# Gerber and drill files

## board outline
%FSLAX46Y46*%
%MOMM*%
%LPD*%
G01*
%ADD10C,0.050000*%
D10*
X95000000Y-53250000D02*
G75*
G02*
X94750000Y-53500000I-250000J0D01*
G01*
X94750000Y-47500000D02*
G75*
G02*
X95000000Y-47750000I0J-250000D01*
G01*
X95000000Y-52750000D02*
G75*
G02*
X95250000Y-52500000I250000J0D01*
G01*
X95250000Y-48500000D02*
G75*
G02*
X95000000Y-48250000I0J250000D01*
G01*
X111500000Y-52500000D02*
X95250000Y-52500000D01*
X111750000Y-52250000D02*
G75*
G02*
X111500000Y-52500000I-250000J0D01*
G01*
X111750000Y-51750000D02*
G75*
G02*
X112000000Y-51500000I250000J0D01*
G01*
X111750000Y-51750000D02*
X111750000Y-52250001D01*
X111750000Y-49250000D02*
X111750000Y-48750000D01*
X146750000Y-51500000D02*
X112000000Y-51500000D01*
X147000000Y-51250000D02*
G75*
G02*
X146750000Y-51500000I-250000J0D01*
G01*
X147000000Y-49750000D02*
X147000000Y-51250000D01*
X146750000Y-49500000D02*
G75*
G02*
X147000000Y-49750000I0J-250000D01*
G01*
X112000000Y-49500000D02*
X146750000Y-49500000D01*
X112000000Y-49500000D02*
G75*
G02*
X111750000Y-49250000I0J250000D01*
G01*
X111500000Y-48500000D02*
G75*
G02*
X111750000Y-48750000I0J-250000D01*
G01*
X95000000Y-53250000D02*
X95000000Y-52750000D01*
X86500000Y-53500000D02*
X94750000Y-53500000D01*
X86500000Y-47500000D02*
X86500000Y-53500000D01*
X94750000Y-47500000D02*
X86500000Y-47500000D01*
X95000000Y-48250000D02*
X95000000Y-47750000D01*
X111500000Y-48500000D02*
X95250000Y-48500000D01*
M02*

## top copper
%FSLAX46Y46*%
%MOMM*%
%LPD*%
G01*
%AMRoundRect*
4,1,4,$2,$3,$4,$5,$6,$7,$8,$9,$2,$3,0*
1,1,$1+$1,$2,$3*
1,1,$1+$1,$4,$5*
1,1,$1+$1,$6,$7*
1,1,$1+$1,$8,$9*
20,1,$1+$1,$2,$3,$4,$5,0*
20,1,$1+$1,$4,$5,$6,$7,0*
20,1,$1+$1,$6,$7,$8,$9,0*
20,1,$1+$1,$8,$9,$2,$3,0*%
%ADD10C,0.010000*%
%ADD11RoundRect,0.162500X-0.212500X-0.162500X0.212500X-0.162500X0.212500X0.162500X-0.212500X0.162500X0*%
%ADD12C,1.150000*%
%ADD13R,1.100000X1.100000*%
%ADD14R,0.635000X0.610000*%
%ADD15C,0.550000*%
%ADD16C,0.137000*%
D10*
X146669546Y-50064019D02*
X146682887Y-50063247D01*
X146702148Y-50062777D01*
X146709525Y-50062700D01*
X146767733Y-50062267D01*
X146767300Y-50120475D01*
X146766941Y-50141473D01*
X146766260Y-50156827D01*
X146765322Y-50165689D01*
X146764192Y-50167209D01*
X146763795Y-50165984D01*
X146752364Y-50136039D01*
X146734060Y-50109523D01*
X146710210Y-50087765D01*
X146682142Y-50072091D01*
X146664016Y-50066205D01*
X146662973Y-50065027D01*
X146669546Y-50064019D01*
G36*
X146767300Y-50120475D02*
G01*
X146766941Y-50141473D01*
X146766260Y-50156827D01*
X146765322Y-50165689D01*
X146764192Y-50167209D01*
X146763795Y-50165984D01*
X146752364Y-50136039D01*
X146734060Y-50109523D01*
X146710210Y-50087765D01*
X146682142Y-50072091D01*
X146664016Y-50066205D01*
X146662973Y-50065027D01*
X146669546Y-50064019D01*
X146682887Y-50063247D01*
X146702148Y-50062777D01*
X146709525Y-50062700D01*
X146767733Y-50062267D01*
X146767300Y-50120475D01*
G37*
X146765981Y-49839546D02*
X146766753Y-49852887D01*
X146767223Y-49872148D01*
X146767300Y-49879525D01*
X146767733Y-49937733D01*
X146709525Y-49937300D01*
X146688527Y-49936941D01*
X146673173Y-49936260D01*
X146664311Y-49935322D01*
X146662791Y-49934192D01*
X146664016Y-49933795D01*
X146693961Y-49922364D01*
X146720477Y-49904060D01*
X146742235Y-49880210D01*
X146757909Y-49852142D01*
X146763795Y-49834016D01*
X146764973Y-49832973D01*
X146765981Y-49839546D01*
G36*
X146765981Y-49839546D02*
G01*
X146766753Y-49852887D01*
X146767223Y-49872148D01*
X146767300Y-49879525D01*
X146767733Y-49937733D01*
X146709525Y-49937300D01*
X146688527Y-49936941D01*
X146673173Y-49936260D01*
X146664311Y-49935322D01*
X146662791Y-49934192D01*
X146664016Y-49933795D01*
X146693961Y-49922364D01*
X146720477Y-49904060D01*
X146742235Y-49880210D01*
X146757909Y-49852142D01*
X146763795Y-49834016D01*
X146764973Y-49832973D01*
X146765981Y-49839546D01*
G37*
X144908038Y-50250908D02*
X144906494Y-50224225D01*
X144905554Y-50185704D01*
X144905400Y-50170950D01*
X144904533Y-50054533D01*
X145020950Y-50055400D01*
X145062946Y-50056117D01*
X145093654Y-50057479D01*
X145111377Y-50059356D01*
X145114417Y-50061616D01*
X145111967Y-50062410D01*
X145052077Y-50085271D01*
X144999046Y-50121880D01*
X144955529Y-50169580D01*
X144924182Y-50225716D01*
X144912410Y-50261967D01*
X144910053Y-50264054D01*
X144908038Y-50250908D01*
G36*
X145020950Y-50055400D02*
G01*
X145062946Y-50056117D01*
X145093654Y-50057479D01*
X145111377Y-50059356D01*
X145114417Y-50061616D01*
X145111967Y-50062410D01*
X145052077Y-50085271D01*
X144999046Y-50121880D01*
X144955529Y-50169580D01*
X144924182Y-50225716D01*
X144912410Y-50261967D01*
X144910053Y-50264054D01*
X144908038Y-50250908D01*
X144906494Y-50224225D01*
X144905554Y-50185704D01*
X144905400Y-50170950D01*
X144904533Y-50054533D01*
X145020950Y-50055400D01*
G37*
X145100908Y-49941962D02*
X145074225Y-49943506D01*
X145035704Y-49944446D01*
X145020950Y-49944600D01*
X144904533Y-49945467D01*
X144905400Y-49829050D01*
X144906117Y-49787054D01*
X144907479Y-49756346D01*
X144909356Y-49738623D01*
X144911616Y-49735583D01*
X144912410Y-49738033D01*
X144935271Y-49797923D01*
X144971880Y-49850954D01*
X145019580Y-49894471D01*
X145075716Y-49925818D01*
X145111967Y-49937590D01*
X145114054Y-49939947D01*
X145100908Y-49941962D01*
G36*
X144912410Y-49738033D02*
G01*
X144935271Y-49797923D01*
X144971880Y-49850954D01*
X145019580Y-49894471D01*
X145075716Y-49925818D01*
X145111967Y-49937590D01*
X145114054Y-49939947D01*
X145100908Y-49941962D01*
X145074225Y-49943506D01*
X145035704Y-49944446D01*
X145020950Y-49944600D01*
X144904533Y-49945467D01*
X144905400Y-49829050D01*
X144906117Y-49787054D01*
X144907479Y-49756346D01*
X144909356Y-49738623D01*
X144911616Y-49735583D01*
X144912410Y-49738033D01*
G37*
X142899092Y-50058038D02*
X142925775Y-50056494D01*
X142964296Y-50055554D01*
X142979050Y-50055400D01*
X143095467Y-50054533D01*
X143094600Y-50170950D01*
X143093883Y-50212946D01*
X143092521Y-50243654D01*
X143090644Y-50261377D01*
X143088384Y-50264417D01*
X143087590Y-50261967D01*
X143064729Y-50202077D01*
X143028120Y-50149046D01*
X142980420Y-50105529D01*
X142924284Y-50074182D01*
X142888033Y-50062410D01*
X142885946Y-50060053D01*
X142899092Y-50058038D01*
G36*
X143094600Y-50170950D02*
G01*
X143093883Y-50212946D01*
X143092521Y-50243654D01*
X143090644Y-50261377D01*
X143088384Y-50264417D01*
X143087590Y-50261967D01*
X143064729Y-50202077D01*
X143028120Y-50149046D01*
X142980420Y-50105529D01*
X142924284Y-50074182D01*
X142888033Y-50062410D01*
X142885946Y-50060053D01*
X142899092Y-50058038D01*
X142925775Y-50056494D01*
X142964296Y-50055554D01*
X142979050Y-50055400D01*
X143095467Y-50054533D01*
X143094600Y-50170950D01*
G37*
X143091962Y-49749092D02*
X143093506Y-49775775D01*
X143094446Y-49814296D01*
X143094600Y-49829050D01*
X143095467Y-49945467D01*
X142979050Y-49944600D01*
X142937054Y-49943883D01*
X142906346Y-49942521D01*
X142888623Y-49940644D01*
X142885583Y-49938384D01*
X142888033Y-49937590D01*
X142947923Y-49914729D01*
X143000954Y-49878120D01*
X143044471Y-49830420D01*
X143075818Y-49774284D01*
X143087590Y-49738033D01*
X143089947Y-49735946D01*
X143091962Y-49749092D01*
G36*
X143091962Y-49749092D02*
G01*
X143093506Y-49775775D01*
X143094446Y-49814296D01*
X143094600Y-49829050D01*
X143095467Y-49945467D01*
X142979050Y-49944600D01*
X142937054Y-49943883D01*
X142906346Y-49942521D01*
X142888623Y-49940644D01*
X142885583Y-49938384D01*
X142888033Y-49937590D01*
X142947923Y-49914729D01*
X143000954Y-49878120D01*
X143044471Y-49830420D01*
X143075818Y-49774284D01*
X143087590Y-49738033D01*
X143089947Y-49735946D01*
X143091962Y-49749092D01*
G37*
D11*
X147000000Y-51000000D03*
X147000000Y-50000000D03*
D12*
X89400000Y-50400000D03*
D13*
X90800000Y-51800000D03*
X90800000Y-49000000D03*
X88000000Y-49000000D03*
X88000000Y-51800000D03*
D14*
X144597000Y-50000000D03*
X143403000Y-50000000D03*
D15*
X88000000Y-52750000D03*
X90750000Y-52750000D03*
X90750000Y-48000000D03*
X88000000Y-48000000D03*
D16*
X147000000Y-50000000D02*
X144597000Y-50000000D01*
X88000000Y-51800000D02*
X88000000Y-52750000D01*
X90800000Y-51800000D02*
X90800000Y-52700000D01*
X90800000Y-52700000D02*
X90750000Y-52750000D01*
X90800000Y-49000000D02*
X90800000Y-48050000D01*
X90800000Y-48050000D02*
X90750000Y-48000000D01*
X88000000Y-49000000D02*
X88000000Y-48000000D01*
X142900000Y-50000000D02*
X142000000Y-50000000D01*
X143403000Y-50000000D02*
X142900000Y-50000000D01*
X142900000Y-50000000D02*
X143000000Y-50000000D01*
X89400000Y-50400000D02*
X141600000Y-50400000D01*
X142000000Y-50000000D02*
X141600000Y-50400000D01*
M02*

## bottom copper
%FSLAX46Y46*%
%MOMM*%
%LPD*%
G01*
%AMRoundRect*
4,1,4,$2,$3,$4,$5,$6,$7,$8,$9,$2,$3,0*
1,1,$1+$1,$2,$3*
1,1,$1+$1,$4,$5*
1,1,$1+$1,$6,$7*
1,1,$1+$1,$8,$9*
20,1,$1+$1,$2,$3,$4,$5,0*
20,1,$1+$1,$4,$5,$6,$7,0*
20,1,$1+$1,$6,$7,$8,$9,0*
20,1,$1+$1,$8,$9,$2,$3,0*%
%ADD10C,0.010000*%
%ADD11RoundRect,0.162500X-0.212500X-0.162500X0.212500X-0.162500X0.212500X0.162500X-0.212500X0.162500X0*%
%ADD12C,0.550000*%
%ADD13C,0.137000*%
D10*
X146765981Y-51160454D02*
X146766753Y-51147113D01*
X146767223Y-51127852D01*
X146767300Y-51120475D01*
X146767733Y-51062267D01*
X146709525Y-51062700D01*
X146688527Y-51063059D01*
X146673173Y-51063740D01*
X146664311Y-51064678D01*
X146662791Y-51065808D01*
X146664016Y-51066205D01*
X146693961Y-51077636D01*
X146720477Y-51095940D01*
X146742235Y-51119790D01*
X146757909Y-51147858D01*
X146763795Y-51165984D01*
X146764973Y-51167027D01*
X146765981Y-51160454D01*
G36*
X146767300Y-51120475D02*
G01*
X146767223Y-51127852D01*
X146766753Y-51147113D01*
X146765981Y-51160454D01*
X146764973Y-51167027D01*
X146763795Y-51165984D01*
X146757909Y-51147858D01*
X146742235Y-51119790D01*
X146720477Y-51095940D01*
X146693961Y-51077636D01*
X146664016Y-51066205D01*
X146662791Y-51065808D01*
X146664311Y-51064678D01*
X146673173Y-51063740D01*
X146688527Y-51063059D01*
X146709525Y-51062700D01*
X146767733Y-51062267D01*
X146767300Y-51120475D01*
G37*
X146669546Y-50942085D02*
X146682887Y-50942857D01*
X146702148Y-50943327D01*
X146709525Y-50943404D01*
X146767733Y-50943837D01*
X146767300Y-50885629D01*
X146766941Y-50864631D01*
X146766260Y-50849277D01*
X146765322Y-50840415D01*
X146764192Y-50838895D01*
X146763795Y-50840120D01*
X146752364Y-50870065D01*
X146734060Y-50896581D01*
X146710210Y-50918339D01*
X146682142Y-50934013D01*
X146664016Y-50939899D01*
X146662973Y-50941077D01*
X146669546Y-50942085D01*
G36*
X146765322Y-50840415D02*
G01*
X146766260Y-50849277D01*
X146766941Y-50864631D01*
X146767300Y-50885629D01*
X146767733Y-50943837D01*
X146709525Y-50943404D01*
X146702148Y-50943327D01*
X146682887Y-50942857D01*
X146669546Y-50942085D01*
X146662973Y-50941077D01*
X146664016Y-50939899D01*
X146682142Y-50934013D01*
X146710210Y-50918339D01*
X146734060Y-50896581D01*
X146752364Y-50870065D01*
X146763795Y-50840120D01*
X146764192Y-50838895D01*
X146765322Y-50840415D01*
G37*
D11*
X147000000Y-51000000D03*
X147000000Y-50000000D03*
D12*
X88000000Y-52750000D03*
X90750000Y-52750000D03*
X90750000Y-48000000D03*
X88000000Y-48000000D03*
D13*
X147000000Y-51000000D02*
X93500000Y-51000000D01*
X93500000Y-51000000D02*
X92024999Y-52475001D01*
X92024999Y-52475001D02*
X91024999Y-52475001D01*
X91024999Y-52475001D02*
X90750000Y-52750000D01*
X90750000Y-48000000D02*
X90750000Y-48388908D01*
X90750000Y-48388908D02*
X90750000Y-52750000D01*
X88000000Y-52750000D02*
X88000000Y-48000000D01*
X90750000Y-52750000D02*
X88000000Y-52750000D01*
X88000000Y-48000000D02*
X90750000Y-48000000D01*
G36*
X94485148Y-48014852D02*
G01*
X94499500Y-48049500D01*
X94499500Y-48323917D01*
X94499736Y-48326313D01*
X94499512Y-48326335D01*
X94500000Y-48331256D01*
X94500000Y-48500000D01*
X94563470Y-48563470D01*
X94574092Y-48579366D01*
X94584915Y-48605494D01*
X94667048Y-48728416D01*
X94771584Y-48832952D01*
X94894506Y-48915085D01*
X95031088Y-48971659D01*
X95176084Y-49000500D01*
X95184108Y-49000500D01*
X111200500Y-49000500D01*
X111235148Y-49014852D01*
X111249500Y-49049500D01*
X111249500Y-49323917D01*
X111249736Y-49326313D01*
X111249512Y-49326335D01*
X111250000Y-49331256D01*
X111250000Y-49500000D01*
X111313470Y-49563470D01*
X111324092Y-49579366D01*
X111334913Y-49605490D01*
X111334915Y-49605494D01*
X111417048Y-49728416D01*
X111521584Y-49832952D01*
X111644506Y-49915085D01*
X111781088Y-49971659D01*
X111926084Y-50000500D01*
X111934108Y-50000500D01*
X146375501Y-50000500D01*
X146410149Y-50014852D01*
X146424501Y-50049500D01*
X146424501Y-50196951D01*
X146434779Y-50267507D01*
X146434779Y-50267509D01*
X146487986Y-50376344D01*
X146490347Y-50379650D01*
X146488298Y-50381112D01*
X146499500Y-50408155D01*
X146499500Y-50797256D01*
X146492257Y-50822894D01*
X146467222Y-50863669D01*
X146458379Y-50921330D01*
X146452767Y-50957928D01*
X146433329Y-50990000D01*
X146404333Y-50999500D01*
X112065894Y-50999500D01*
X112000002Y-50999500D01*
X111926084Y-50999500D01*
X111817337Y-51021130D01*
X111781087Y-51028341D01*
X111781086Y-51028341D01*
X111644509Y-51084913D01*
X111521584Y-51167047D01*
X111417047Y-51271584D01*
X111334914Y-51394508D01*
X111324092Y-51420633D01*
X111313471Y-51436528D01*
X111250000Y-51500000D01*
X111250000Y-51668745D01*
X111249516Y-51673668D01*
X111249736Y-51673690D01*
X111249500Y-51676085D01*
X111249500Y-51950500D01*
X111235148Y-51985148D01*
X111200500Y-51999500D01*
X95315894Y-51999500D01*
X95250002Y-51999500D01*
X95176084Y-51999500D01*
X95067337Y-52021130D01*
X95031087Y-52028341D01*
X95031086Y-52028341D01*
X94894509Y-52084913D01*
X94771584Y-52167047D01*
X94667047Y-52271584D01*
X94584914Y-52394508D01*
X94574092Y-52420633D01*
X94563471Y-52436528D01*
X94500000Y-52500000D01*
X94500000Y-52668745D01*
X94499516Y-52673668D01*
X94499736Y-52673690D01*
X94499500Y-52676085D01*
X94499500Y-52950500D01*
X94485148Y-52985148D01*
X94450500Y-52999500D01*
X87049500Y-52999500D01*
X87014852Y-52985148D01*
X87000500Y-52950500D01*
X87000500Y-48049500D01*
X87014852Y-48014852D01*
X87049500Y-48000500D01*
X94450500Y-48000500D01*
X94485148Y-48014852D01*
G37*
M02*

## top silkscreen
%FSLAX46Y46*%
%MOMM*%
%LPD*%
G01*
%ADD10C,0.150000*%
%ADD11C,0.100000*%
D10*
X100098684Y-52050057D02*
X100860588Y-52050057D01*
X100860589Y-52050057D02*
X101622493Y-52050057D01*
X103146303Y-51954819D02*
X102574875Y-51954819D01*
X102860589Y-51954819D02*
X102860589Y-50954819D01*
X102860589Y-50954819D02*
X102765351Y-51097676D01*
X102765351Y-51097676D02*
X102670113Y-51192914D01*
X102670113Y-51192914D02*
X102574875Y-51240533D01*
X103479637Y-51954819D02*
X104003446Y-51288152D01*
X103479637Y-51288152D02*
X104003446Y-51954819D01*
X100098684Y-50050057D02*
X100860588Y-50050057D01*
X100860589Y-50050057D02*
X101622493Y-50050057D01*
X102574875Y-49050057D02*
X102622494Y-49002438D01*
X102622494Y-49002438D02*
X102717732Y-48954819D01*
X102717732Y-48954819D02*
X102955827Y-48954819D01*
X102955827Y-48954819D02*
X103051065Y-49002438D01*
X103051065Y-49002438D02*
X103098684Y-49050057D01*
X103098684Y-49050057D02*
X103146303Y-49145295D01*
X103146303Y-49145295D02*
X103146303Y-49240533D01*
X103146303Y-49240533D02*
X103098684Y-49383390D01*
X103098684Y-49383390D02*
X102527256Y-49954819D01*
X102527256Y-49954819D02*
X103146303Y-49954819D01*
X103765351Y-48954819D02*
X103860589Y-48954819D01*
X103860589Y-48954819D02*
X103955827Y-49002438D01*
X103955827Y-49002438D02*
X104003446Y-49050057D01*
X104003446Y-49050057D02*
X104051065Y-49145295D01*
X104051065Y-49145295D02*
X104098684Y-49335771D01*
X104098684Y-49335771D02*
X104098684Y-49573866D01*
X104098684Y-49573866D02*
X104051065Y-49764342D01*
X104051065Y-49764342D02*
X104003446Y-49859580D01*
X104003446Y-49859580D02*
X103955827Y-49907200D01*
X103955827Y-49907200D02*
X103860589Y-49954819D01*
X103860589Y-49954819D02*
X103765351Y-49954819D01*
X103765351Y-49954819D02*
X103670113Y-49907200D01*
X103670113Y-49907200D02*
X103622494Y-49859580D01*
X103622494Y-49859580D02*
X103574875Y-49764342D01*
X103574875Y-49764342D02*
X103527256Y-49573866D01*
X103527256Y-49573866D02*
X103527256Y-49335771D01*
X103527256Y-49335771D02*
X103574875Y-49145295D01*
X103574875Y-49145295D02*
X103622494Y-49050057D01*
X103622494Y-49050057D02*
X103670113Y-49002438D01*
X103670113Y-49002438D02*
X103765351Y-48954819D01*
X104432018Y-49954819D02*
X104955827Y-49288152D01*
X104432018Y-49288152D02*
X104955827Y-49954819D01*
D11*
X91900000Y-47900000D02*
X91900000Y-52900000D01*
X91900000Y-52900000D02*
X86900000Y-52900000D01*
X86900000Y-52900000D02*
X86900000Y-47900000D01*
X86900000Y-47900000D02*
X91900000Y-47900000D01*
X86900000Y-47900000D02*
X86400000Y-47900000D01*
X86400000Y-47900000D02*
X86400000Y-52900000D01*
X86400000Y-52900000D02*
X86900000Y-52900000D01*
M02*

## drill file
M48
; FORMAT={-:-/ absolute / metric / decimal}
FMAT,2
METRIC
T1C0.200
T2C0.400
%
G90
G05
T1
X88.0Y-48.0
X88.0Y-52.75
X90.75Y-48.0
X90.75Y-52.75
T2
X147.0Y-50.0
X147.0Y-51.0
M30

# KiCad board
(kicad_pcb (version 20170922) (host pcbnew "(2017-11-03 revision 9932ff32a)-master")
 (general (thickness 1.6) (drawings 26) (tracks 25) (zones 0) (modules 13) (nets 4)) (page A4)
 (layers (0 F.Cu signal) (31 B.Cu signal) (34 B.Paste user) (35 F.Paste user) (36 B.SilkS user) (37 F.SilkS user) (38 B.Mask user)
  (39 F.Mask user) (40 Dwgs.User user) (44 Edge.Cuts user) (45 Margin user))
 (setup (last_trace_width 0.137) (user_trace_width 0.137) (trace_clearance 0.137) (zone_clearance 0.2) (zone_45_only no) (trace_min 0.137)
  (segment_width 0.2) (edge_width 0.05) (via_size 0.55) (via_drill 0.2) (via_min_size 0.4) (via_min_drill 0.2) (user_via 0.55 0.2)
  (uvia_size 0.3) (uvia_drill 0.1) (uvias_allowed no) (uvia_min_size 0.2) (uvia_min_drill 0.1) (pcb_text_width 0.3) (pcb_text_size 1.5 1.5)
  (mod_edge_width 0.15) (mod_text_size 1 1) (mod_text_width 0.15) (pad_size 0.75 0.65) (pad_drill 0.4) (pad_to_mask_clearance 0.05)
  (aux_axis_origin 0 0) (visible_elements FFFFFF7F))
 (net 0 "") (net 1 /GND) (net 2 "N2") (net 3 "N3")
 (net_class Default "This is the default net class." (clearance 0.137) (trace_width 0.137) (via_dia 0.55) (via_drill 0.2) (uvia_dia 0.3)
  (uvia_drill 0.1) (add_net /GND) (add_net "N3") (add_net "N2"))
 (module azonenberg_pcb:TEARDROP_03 (layer B.Cu) (at 146.7 51.13)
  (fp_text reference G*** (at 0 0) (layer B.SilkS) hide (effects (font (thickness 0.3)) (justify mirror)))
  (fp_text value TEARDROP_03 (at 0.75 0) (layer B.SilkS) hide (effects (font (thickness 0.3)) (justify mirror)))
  (fp_poly
   (pts (xy 0.065981 0.030454) (xy 0.066753 0.017113) (xy 0.067223 -0.002148) (xy 0.0673 -0.009525) (xy 0.067733 -0.067733)
    (xy 0.009525 -0.0673) (xy -0.011473 -0.066941) (xy -0.026827 -0.06626) (xy -0.035689 -0.065322) (xy -0.037209 -0.064192)
    (xy -0.035984 -0.063795) (xy -0.006039 -0.052364) (xy 0.020477 -0.03406) (xy 0.042235 -0.01021) (xy 0.057909 0.017858)
    (xy 0.063795 0.035984) (xy 0.064973 0.037027) (xy 0.065981 0.030454))
   (layer B.Cu) (width 0.01)))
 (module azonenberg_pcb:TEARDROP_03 (layer B.Cu) (at 146.7 50.876104 270)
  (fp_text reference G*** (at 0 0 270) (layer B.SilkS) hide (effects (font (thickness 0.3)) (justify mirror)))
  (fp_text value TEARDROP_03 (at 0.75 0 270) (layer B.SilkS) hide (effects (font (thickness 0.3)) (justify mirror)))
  (fp_poly
   (pts (xy 0.065981 0.030454) (xy 0.066753 0.017113) (xy 0.067223 -0.002148) (xy 0.0673 -0.009525) (xy 0.067733 -0.067733)
    (xy 0.009525 -0.0673) (xy -0.011473 -0.066941) (xy -0.026827 -0.06626) (xy -0.035689 -0.065322) (xy -0.037209 -0.064192)
    (xy -0.035984 -0.063795) (xy -0.006039 -0.052364) (xy 0.020477 -0.03406) (xy 0.042235 -0.01021) (xy 0.057909 0.017858)
    (xy 0.063795 0.035984) (xy 0.064973 0.037027) (xy 0.065981 0.030454))
   (layer B.Cu) (width 0.01)))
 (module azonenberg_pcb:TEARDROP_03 (layer F.Cu) (at 146.7 50.13 90)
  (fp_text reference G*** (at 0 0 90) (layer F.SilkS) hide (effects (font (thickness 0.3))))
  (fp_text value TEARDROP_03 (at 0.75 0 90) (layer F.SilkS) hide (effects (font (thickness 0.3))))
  (fp_poly
   (pts (xy 0.065981 -0.030454) (xy 0.066753 -0.017113) (xy 0.067223 0.002148) (xy 0.0673 0.009525) (xy 0.067733 0.067733)
    (xy 0.009525 0.0673) (xy -0.011473 0.066941) (xy -0.026827 0.06626) (xy -0.035689 0.065322) (xy -0.037209 0.064192)
    (xy -0.035984 0.063795) (xy -0.006039 0.052364) (xy 0.020477 0.03406) (xy 0.042235 0.01021) (xy 0.057909 -0.017858)
    (xy 0.063795 -0.035984) (xy 0.064973 -0.037027) (xy 0.065981 -0.030454))
   (layer F.Cu) (width 0.01)))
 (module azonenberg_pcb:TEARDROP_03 (layer F.Cu) (at 146.7 49.87)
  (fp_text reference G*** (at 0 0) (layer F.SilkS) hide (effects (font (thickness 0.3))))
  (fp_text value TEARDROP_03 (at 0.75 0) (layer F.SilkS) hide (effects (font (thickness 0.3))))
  (fp_poly
   (pts (xy 0.065981 -0.030454) (xy 0.066753 -0.017113) (xy 0.067223 0.002148) (xy 0.0673 0.009525) (xy 0.067733 0.067733)
    (xy 0.009525 0.0673) (xy -0.011473 0.066941) (xy -0.026827 0.06626) (xy -0.035689 0.065322) (xy -0.037209 0.064192)
    (xy -0.035984 0.063795) (xy -0.006039 0.052364) (xy 0.020477 0.03406) (xy 0.042235 0.01021) (xy 0.057909 -0.017858)
    (xy 0.063795 -0.035984) (xy 0.064973 -0.037027) (xy 0.065981 -0.030454))
   (layer F.Cu) (width 0.01)))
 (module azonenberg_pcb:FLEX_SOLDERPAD (layer F.Cu) (at 147 51)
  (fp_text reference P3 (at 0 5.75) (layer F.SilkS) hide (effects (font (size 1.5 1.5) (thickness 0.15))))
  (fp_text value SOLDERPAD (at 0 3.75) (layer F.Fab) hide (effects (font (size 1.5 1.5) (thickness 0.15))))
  (pad 1 thru_hole roundrect (at 0 0) (size 0.75 0.65) (drill 0.4) (layers *.Cu *.Mask) (roundrect_rratio 0.25) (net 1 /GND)))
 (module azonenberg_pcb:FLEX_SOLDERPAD (layer F.Cu) (at 147 50)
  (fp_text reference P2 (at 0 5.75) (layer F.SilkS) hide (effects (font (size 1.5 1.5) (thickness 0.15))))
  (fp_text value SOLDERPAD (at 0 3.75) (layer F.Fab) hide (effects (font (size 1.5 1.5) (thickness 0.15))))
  (pad 1 thru_hole roundrect (at 0 0) (size 0.75 0.65) (drill 0.4) (layers *.Cu *.Mask) (roundrect_rratio 0.25) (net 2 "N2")))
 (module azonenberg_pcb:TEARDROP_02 (layer F.Cu) (at 145.04 50.19 180)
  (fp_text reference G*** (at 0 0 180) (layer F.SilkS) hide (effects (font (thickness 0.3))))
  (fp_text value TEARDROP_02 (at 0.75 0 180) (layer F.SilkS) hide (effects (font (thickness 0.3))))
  (fp_poly
   (pts (xy 0.131962 -0.060908) (xy 0.133506 -0.034225) (xy 0.134446 0.004296) (xy 0.1346 0.01905) (xy 0.135467 0.135467)
    (xy 0.01905 0.1346) (xy -0.022946 0.133883) (xy -0.053654 0.132521) (xy -0.071377 0.130644) (xy -0.074417 0.128384)
    (xy -0.071967 0.12759) (xy -0.012077 0.104729) (xy 0.040954 0.06812) (xy 0.084471 0.02042) (xy 0.115818 -0.035716)
    (xy 0.12759 -0.071967) (xy 0.129947 -0.074054) (xy 0.131962 -0.060908))
   (layer F.Cu) (width 0.01)))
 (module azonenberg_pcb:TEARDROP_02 (layer F.Cu) (at 145.04 49.81 270)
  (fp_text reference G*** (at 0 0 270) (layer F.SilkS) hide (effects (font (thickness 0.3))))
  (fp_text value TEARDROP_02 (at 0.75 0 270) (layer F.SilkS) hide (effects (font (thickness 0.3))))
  (fp_poly
   (pts (xy 0.131962 -0.060908) (xy 0.133506 -0.034225) (xy 0.134446 0.004296) (xy 0.1346 0.01905) (xy 0.135467 0.135467)
    (xy 0.01905 0.1346) (xy -0.022946 0.133883) (xy -0.053654 0.132521) (xy -0.071377 0.130644) (xy -0.074417 0.128384)
    (xy -0.071967 0.12759) (xy -0.012077 0.104729) (xy 0.040954 0.06812) (xy 0.084471 0.02042) (xy 0.115818 -0.035716)
    (xy 0.12759 -0.071967) (xy 0.129947 -0.074054) (xy 0.131962 -0.060908))
   (layer F.Cu) (width 0.01)))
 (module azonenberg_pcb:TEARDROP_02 (layer F.Cu) (at 142.96 50.19 90)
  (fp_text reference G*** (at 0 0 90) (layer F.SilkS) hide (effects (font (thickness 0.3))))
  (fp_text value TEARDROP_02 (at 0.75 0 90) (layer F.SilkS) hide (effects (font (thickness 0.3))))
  (fp_poly
   (pts (xy 0.131962 -0.060908) (xy 0.133506 -0.034225) (xy 0.134446 0.004296) (xy 0.1346 0.01905) (xy 0.135467 0.135467)
    (xy 0.01905 0.1346) (xy -0.022946 0.133883) (xy -0.053654 0.132521) (xy -0.071377 0.130644) (xy -0.074417 0.128384)
    (xy -0.071967 0.12759) (xy -0.012077 0.104729) (xy 0.040954 0.06812) (xy 0.084471 0.02042) (xy 0.115818 -0.035716)
    (xy 0.12759 -0.071967) (xy 0.129947 -0.074054) (xy 0.131962 -0.060908))
   (layer F.Cu) (width 0.01)))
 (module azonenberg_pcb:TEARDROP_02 (layer F.Cu) (at 142.96 49.81)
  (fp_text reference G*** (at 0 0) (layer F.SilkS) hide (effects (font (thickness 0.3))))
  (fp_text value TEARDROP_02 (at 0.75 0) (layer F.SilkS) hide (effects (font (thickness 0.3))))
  (fp_poly
   (pts (xy 0.131962 -0.060908) (xy 0.133506 -0.034225) (xy 0.134446 0.004296) (xy 0.1346 0.01905) (xy 0.135467 0.135467)
    (xy 0.01905 0.1346) (xy -0.022946 0.133883) (xy -0.053654 0.132521) (xy -0.071377 0.130644) (xy -0.074417 0.128384)
    (xy -0.071967 0.12759) (xy -0.012077 0.104729) (xy 0.040954 0.06812) (xy 0.084471 0.02042) (xy 0.115818 -0.035716)
    (xy 0.12759 -0.071967) (xy 0.129947 -0.074054) (xy 0.131962 -0.060908))
   (layer F.Cu) (width 0.01)))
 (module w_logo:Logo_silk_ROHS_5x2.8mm (layer B.Cu) (at 93.25 50.5 270)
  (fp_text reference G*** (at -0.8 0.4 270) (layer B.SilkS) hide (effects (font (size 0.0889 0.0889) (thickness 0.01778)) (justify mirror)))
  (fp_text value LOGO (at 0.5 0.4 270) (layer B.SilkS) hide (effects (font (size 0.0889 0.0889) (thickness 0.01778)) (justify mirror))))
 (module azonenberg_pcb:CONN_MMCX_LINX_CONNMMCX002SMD (layer F.Cu) (at 89.4 50.4)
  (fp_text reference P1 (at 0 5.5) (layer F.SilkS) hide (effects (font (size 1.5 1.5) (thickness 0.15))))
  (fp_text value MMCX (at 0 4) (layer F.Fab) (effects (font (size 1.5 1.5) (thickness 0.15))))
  (fp_line (start 2.5 -2.5) (end 2.5 2.5) (layer F.SilkS) (width 0.1))
  (fp_line (start 2.5 2.5) (end -2.5 2.5) (layer F.SilkS) (width 0.1))
  (fp_line (start -2.5 2.5) (end -2.5 -2.5) (layer F.SilkS) (width 0.1))
  (fp_line (start -2.5 -2.5) (end 2.5 -2.5) (layer F.SilkS) (width 0.1))
  (fp_line (start -2.5 -2.5) (end -3 -2.5) (layer F.SilkS) (width 0.1))
  (fp_line (start -3 -2.5) (end -3 2.5) (layer F.SilkS) (width 0.1))
  (fp_line (start -3 2.5) (end -2.5 2.5) (layer F.SilkS) (width 0.1))
  (pad 1 smd circle (at 0 0) (size 1.15 1.15) (layers F.Cu F.Paste F.Mask) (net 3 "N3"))
  (pad 2 smd rect (at 1.4 1.4) (size 1.1 1.1) (layers F.Cu F.Paste F.Mask) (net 1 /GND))
  (pad 2 smd rect (at 1.4 -1.4) (size 1.1 1.1) (layers F.Cu F.Paste F.Mask) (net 1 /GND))
  (pad 2 smd rect (at -1.4 -1.4) (size 1.1 1.1) (layers F.Cu F.Paste F.Mask) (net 1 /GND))
  (pad 2 smd rect (at -1.4 1.4) (size 1.1 1.1) (layers F.Cu F.Paste F.Mask) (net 1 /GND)))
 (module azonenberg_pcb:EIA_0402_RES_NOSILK (layer F.Cu) (at 144 50 180)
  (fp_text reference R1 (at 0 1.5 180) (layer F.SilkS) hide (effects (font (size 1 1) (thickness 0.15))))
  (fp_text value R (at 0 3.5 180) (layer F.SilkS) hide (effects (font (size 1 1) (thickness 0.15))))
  (pad 1 smd rect (at -0.597 0 180) (size 0.635 0.61) (layers F.Cu F.Paste F.Mask) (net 2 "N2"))
  (pad 2 smd rect (at 0.597 0 180) (size 0.635 0.61) (layers F.Cu F.Paste F.Mask) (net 3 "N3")))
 (gr_arc (start 94.75 53.25) (end 94.75 53.5) (angle -90) (layer Edge.Cuts) (width 0.05))
 (gr_arc (start 94.75 47.75) (end 95 47.75) (angle -90) (layer Edge.Cuts) (width 0.05))
 (gr_arc (start 95.25 52.75) (end 95.25 52.5) (angle -90) (layer Edge.Cuts) (width 0.05))
 (gr_arc (start 95.25 48.25) (end 95 48.25) (angle -90) (layer Edge.Cuts) (width 0.05))
 (gr_line (start 111.5 52.5) (end 95.25 52.5) (layer Edge.Cuts) (width 0.05))
 (gr_arc (start 111.5 52.25) (end 111.5 52.5) (angle -90) (layer Edge.Cuts) (width 0.05))
 (gr_arc (start 112 51.75) (end 112 51.5) (angle -90) (layer Edge.Cuts) (width 0.05))
 (gr_line (start 111.75 51.75) (end 111.75 52.250001) (layer Edge.Cuts) (width 0.05))
 (gr_line (start 111.75 49.25) (end 111.75 48.75) (layer Edge.Cuts) (width 0.05))
 (gr_line (start 146.75 51.5) (end 112 51.5) (layer Edge.Cuts) (width 0.05))
 (gr_arc (start 146.75 51.25) (end 146.75 51.5) (angle -90) (layer Edge.Cuts) (width 0.05))
 (gr_line (start 147 49.75) (end 147 51.25) (layer Edge.Cuts) (width 0.05))
 (gr_arc (start 146.75 49.75) (end 147 49.75) (angle -90) (layer Edge.Cuts) (width 0.05))
 (gr_line (start 112 49.5) (end 146.75 49.5) (layer Edge.Cuts) (width 0.05))
 (gr_arc (start 112 49.25) (end 111.75 49.25) (angle -90) (layer Edge.Cuts) (width 0.05))
 (gr_arc (start 111.5 48.75) (end 111.75 48.75) (angle -90) (layer Edge.Cuts) (width 0.05))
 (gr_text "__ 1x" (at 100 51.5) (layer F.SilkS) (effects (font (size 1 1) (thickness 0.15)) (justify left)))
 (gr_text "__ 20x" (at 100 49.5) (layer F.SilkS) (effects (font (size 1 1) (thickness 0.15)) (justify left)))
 (gr_line (start 95 53.25) (end 95 52.75) (layer Edge.Cuts) (width 0.05))
 (gr_line (start 86.5 53.5) (end 94.75 53.5) (layer Edge.Cuts) (width 0.05))
 (gr_line (start 86.5 47.5) (end 86.5 53.5) (layer Edge.Cuts) (width 0.05))
 (gr_line (start 94.75 47.5) (end 86.5 47.5) (layer Edge.Cuts) (width 0.05))
 (gr_line (start 95 48.25) (end 95 47.75) (layer Edge.Cuts) (width 0.05))
 (gr_line (start 111.5 48.5) (end 95.25 48.5) (layer Edge.Cuts) (width 0.05))
 (segment (start 147 50) (end 144.597 50) (width 0.137) (layer F.Cu) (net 2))
 (segment (start 147 51) (end 93.5 51) (width 0.137) (layer B.Cu) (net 1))
 (segment (start 93.5 51) (end 92.024999 52.475001) (width 0.137) (layer B.Cu) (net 1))
 (segment (start 92.024999 52.475001) (end 91.024999 52.475001) (width 0.137) (layer B.Cu) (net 1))
 (segment (start 91.024999 52.475001) (end 90.75 52.75) (width 0.137) (layer B.Cu) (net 1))
 (segment (start 90.75 48) (end 90.75 48.388908) (width 0.137) (layer B.Cu) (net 1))
 (segment (start 90.75 48.388908) (end 90.75 52.75) (width 0.137) (layer B.Cu) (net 1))
 (segment (start 88 52.75) (end 88 48) (width 0.137) (layer B.Cu) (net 1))
 (segment (start 90.75 52.75) (end 88 52.75) (width 0.137) (layer B.Cu) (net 1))
 (segment (start 88 48) (end 90.75 48) (width 0.137) (layer B.Cu) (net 1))
 (segment (start 88 51.8) (end 88 52.75) (width 0.137) (layer F.Cu) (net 1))
 (via (at 88 52.75) (size 0.55) (drill 0.2) (layers F.Cu B.Cu) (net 1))
 (segment (start 90.8 51.8) (end 90.8 52.7) (width 0.137) (layer F.Cu) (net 1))
 (segment (start 90.8 52.7) (end 90.75 52.75) (width 0.137) (layer F.Cu) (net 1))
 (via (at 90.75 52.75) (size 0.55) (drill 0.2) (layers F.Cu B.Cu) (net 1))
 (segment (start 90.8 49) (end 90.8 48.05) (width 0.137) (layer F.Cu) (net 1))
 (segment (start 90.8 48.05) (end 90.75 48) (width 0.137) (layer F.Cu) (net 1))
 (via (at 90.75 48) (size 0.55) (drill 0.2) (layers F.Cu B.Cu) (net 1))
 (segment (start 88 49) (end 88 48) (width 0.137) (layer F.Cu) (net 1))
 (via (at 88 48) (size 0.55) (drill 0.2) (layers F.Cu B.Cu) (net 1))
 (segment (start 142.9 50) (end 142 50) (width 0.137) (layer F.Cu) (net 3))
 (segment (start 143.403 50) (end 142.9 50) (width 0.137) (layer F.Cu) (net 3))
 (segment (start 142.9 50) (end 143 50) (width 0.137) (layer F.Cu) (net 3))
 (segment (start 89.4 50.4) (end 141.6 50.4) (width 0.137) (layer F.Cu) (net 3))
 (segment (start 142 50) (end 141.6 50.4) (width 0.137) (layer F.Cu) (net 3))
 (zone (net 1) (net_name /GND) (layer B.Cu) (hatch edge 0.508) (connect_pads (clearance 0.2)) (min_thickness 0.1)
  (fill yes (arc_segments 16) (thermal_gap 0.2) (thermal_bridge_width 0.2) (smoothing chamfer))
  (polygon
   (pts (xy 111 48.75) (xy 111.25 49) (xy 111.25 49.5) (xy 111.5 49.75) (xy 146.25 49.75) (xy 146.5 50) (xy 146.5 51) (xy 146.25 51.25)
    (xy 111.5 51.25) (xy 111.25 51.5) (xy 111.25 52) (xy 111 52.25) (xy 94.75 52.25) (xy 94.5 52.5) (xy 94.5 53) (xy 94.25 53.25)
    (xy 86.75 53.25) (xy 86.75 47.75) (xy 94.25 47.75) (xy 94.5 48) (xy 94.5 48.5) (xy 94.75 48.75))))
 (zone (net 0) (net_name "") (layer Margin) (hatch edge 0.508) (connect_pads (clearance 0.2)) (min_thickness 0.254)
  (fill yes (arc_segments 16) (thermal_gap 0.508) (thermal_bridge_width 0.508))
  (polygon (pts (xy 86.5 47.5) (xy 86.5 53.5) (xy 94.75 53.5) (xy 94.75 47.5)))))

